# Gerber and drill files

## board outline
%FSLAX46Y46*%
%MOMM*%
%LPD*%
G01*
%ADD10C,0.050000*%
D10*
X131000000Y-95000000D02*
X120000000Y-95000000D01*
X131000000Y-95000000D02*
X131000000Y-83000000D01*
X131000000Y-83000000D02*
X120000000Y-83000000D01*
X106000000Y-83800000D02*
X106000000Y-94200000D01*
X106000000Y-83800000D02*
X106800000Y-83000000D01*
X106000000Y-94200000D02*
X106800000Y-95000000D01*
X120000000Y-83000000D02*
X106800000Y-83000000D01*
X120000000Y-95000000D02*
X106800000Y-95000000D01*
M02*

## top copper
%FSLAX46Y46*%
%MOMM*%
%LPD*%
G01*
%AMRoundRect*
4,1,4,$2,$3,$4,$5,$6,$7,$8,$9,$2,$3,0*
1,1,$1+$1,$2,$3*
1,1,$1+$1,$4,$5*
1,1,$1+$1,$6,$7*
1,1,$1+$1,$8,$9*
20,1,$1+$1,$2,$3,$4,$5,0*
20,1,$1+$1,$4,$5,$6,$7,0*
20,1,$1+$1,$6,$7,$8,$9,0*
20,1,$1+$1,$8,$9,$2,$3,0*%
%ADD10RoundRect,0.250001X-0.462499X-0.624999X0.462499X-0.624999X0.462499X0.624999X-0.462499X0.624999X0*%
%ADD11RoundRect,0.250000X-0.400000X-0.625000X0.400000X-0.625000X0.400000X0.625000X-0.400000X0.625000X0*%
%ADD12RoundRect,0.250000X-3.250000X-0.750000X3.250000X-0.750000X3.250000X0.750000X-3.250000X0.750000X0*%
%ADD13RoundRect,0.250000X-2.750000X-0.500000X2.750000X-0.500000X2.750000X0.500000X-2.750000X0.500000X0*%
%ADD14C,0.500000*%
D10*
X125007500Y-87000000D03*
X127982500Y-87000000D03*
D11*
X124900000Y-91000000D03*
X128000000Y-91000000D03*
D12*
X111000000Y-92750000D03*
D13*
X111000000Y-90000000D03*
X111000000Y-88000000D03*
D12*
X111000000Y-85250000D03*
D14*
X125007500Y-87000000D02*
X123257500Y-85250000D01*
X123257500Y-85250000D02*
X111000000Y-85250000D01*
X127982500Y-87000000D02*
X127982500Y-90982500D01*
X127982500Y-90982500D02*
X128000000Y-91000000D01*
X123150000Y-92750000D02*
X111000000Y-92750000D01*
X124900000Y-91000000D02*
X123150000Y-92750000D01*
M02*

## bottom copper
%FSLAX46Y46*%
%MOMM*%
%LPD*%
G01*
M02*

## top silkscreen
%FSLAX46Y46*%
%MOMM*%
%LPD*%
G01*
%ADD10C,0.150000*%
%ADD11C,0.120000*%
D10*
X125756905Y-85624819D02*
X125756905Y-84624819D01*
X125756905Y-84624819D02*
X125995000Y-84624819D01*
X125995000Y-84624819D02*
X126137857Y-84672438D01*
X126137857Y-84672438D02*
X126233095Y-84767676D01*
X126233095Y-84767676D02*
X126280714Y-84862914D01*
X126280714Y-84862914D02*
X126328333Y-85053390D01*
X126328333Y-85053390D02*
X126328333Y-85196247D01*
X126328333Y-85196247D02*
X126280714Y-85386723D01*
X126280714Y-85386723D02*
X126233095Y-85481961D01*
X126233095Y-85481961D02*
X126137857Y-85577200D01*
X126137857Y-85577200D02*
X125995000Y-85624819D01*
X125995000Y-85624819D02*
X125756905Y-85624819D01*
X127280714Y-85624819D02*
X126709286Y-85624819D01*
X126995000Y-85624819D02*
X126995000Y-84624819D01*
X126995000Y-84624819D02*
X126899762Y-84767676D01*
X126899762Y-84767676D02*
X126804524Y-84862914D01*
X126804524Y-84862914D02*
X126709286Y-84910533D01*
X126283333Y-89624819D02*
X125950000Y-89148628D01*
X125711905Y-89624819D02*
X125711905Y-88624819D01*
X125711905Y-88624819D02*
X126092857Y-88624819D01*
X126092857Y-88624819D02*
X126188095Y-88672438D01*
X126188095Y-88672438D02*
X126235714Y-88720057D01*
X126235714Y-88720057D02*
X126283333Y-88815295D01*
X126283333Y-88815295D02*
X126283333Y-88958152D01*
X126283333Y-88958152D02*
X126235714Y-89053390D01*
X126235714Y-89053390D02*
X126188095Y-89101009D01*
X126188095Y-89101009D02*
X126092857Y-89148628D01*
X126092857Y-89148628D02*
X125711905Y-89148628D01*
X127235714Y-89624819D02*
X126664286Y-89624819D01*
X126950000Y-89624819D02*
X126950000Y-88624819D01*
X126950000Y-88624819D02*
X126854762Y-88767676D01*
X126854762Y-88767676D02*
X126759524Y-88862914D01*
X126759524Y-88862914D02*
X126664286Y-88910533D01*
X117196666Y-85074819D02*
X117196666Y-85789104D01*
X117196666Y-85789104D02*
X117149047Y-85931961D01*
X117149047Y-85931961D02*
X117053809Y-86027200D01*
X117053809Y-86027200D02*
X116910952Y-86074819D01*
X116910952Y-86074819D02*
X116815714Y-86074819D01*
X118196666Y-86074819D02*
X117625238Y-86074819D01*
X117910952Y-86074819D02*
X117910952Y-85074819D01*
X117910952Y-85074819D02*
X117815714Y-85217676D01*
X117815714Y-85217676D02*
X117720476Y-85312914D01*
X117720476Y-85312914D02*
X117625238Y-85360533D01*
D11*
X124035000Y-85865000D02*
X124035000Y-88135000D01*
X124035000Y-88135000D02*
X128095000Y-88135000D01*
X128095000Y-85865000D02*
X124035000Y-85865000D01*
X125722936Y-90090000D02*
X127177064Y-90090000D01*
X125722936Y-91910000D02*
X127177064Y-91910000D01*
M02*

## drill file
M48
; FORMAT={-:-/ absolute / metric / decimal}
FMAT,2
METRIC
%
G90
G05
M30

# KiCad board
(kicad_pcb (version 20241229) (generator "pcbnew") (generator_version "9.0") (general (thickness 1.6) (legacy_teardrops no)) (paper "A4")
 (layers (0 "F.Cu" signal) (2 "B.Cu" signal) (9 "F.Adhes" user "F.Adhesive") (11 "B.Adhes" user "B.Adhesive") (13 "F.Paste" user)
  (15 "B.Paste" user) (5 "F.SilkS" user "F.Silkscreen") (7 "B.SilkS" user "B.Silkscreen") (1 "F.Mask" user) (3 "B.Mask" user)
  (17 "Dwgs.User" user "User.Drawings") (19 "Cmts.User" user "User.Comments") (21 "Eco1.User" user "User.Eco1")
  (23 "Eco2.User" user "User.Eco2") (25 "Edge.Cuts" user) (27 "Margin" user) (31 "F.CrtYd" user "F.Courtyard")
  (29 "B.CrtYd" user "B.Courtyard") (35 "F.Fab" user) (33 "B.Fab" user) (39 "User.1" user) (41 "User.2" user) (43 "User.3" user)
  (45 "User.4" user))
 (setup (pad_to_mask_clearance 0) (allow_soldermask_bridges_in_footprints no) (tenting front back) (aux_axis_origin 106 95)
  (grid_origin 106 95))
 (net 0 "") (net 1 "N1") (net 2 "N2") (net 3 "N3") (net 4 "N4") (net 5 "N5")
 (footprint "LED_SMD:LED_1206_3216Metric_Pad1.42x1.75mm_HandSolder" (layer "F.Cu") (at 126.495 87)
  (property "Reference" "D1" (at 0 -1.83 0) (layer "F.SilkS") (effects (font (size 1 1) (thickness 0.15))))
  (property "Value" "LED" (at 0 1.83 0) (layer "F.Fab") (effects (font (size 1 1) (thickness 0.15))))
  (fp_line (start -2.46 -1.135) (end -2.46 1.135) (stroke (width 0.12) (type solid)) (layer "F.SilkS"))
  (fp_line (start -2.46 1.135) (end 1.6 1.135) (stroke (width 0.12) (type solid)) (layer "F.SilkS"))
  (fp_line (start 1.6 -1.135) (end -2.46 -1.135) (stroke (width 0.12) (type solid)) (layer "F.SilkS"))
  (pad "1" smd roundrect (at -1.4875 0) (size 1.425 1.75) (layers "F.Cu" "F.Mask" "F.Paste") (roundrect_rratio 0.175439) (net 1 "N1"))
  (pad "2" smd roundrect (at 1.4875 0) (size 1.425 1.75) (layers "F.Cu" "F.Mask" "F.Paste") (roundrect_rratio 0.175439) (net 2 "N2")))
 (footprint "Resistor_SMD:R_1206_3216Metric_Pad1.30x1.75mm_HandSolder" (layer "F.Cu") (at 126.45 91)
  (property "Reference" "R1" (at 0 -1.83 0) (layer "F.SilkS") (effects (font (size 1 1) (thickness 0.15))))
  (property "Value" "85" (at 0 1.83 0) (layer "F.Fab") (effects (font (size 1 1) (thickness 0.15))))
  (fp_line (start -0.727064 -0.91) (end 0.727064 -0.91) (stroke (width 0.12) (type solid)) (layer "F.SilkS"))
  (fp_line (start -0.727064 0.91) (end 0.727064 0.91) (stroke (width 0.12) (type solid)) (layer "F.SilkS"))
  (pad "1" smd roundrect (at -1.55 0) (size 1.3 1.75) (layers "F.Cu" "F.Mask" "F.Paste") (roundrect_rratio 0.192308) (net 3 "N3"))
  (pad "2" smd roundrect (at 1.55 0) (size 1.3 1.75) (layers "F.Cu" "F.Mask" "F.Paste") (roundrect_rratio 0.192308) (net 2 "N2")))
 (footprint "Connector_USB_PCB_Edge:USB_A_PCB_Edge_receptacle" (layer "F.Cu") (at 111 89)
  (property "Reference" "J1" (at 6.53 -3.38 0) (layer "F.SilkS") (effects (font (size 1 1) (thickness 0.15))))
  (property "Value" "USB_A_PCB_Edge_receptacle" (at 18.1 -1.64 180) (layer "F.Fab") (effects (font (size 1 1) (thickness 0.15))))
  (fp_line (start -5 -5.2) (end -5 5.2) (stroke (width 0.05) (type default)) (layer "Edge.Cuts"))
  (fp_line (start -5 -5.2) (end -4.2 -6) (stroke (width 0.05) (type default)) (layer "Edge.Cuts"))
  (fp_line (start -5 5.2) (end -4.2 6) (stroke (width 0.05) (type default)) (layer "Edge.Cuts"))
  (fp_line (start 9 -6) (end -4.2 -6) (stroke (width 0.05) (type default)) (layer "Edge.Cuts"))
  (fp_line (start 9 6) (end -4.2 6) (stroke (width 0.05) (type default)) (layer "Edge.Cuts"))
  (pad "1" smd roundrect (at 0 3.75) (size 7 2) (layers "F.Cu" "F.Mask") (roundrect_rratio 0.125) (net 3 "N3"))
  (pad "2" smd roundrect (at 0 1) (size 6 1.5) (layers "F.Cu" "F.Mask") (roundrect_rratio 0.1666666667) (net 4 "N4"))
  (pad "3" smd roundrect (at 0 -1) (size 6 1.5) (layers "F.Cu" "F.Mask") (roundrect_rratio 0.1666666667) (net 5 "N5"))
  (pad "4" smd roundrect (at 0 -3.75) (size 7 2) (layers "F.Cu" "F.Mask") (roundrect_rratio 0.125) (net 1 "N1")))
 (gr_line (start 131 95) (end 120 95) (stroke (width 0.05) (type default)) (layer "Edge.Cuts"))
 (gr_line (start 131 95) (end 131 83) (stroke (width 0.05) (type default)) (layer "Edge.Cuts"))
 (gr_line (start 131 83) (end 120 83) (stroke (width 0.05) (type default)) (layer "Edge.Cuts"))
 (segment (start 125.0075 87) (end 123.2575 85.25) (width 0.5) (layer "F.Cu") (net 1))
 (segment (start 123.2575 85.25) (end 111 85.25) (width 0.5) (layer "F.Cu") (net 1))
 (segment (start 127.9825 87) (end 127.9825 90.9825) (width 0.5) (layer "F.Cu") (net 2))
 (segment (start 127.9825 90.9825) (end 128 91) (width 0.5) (layer "F.Cu") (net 2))
 (segment (start 123.15 92.75) (end 111 92.75) (width 0.5) (layer "F.Cu") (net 3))
 (segment (start 124.9 91) (end 123.15 92.75) (width 0.5) (layer "F.Cu") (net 3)))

